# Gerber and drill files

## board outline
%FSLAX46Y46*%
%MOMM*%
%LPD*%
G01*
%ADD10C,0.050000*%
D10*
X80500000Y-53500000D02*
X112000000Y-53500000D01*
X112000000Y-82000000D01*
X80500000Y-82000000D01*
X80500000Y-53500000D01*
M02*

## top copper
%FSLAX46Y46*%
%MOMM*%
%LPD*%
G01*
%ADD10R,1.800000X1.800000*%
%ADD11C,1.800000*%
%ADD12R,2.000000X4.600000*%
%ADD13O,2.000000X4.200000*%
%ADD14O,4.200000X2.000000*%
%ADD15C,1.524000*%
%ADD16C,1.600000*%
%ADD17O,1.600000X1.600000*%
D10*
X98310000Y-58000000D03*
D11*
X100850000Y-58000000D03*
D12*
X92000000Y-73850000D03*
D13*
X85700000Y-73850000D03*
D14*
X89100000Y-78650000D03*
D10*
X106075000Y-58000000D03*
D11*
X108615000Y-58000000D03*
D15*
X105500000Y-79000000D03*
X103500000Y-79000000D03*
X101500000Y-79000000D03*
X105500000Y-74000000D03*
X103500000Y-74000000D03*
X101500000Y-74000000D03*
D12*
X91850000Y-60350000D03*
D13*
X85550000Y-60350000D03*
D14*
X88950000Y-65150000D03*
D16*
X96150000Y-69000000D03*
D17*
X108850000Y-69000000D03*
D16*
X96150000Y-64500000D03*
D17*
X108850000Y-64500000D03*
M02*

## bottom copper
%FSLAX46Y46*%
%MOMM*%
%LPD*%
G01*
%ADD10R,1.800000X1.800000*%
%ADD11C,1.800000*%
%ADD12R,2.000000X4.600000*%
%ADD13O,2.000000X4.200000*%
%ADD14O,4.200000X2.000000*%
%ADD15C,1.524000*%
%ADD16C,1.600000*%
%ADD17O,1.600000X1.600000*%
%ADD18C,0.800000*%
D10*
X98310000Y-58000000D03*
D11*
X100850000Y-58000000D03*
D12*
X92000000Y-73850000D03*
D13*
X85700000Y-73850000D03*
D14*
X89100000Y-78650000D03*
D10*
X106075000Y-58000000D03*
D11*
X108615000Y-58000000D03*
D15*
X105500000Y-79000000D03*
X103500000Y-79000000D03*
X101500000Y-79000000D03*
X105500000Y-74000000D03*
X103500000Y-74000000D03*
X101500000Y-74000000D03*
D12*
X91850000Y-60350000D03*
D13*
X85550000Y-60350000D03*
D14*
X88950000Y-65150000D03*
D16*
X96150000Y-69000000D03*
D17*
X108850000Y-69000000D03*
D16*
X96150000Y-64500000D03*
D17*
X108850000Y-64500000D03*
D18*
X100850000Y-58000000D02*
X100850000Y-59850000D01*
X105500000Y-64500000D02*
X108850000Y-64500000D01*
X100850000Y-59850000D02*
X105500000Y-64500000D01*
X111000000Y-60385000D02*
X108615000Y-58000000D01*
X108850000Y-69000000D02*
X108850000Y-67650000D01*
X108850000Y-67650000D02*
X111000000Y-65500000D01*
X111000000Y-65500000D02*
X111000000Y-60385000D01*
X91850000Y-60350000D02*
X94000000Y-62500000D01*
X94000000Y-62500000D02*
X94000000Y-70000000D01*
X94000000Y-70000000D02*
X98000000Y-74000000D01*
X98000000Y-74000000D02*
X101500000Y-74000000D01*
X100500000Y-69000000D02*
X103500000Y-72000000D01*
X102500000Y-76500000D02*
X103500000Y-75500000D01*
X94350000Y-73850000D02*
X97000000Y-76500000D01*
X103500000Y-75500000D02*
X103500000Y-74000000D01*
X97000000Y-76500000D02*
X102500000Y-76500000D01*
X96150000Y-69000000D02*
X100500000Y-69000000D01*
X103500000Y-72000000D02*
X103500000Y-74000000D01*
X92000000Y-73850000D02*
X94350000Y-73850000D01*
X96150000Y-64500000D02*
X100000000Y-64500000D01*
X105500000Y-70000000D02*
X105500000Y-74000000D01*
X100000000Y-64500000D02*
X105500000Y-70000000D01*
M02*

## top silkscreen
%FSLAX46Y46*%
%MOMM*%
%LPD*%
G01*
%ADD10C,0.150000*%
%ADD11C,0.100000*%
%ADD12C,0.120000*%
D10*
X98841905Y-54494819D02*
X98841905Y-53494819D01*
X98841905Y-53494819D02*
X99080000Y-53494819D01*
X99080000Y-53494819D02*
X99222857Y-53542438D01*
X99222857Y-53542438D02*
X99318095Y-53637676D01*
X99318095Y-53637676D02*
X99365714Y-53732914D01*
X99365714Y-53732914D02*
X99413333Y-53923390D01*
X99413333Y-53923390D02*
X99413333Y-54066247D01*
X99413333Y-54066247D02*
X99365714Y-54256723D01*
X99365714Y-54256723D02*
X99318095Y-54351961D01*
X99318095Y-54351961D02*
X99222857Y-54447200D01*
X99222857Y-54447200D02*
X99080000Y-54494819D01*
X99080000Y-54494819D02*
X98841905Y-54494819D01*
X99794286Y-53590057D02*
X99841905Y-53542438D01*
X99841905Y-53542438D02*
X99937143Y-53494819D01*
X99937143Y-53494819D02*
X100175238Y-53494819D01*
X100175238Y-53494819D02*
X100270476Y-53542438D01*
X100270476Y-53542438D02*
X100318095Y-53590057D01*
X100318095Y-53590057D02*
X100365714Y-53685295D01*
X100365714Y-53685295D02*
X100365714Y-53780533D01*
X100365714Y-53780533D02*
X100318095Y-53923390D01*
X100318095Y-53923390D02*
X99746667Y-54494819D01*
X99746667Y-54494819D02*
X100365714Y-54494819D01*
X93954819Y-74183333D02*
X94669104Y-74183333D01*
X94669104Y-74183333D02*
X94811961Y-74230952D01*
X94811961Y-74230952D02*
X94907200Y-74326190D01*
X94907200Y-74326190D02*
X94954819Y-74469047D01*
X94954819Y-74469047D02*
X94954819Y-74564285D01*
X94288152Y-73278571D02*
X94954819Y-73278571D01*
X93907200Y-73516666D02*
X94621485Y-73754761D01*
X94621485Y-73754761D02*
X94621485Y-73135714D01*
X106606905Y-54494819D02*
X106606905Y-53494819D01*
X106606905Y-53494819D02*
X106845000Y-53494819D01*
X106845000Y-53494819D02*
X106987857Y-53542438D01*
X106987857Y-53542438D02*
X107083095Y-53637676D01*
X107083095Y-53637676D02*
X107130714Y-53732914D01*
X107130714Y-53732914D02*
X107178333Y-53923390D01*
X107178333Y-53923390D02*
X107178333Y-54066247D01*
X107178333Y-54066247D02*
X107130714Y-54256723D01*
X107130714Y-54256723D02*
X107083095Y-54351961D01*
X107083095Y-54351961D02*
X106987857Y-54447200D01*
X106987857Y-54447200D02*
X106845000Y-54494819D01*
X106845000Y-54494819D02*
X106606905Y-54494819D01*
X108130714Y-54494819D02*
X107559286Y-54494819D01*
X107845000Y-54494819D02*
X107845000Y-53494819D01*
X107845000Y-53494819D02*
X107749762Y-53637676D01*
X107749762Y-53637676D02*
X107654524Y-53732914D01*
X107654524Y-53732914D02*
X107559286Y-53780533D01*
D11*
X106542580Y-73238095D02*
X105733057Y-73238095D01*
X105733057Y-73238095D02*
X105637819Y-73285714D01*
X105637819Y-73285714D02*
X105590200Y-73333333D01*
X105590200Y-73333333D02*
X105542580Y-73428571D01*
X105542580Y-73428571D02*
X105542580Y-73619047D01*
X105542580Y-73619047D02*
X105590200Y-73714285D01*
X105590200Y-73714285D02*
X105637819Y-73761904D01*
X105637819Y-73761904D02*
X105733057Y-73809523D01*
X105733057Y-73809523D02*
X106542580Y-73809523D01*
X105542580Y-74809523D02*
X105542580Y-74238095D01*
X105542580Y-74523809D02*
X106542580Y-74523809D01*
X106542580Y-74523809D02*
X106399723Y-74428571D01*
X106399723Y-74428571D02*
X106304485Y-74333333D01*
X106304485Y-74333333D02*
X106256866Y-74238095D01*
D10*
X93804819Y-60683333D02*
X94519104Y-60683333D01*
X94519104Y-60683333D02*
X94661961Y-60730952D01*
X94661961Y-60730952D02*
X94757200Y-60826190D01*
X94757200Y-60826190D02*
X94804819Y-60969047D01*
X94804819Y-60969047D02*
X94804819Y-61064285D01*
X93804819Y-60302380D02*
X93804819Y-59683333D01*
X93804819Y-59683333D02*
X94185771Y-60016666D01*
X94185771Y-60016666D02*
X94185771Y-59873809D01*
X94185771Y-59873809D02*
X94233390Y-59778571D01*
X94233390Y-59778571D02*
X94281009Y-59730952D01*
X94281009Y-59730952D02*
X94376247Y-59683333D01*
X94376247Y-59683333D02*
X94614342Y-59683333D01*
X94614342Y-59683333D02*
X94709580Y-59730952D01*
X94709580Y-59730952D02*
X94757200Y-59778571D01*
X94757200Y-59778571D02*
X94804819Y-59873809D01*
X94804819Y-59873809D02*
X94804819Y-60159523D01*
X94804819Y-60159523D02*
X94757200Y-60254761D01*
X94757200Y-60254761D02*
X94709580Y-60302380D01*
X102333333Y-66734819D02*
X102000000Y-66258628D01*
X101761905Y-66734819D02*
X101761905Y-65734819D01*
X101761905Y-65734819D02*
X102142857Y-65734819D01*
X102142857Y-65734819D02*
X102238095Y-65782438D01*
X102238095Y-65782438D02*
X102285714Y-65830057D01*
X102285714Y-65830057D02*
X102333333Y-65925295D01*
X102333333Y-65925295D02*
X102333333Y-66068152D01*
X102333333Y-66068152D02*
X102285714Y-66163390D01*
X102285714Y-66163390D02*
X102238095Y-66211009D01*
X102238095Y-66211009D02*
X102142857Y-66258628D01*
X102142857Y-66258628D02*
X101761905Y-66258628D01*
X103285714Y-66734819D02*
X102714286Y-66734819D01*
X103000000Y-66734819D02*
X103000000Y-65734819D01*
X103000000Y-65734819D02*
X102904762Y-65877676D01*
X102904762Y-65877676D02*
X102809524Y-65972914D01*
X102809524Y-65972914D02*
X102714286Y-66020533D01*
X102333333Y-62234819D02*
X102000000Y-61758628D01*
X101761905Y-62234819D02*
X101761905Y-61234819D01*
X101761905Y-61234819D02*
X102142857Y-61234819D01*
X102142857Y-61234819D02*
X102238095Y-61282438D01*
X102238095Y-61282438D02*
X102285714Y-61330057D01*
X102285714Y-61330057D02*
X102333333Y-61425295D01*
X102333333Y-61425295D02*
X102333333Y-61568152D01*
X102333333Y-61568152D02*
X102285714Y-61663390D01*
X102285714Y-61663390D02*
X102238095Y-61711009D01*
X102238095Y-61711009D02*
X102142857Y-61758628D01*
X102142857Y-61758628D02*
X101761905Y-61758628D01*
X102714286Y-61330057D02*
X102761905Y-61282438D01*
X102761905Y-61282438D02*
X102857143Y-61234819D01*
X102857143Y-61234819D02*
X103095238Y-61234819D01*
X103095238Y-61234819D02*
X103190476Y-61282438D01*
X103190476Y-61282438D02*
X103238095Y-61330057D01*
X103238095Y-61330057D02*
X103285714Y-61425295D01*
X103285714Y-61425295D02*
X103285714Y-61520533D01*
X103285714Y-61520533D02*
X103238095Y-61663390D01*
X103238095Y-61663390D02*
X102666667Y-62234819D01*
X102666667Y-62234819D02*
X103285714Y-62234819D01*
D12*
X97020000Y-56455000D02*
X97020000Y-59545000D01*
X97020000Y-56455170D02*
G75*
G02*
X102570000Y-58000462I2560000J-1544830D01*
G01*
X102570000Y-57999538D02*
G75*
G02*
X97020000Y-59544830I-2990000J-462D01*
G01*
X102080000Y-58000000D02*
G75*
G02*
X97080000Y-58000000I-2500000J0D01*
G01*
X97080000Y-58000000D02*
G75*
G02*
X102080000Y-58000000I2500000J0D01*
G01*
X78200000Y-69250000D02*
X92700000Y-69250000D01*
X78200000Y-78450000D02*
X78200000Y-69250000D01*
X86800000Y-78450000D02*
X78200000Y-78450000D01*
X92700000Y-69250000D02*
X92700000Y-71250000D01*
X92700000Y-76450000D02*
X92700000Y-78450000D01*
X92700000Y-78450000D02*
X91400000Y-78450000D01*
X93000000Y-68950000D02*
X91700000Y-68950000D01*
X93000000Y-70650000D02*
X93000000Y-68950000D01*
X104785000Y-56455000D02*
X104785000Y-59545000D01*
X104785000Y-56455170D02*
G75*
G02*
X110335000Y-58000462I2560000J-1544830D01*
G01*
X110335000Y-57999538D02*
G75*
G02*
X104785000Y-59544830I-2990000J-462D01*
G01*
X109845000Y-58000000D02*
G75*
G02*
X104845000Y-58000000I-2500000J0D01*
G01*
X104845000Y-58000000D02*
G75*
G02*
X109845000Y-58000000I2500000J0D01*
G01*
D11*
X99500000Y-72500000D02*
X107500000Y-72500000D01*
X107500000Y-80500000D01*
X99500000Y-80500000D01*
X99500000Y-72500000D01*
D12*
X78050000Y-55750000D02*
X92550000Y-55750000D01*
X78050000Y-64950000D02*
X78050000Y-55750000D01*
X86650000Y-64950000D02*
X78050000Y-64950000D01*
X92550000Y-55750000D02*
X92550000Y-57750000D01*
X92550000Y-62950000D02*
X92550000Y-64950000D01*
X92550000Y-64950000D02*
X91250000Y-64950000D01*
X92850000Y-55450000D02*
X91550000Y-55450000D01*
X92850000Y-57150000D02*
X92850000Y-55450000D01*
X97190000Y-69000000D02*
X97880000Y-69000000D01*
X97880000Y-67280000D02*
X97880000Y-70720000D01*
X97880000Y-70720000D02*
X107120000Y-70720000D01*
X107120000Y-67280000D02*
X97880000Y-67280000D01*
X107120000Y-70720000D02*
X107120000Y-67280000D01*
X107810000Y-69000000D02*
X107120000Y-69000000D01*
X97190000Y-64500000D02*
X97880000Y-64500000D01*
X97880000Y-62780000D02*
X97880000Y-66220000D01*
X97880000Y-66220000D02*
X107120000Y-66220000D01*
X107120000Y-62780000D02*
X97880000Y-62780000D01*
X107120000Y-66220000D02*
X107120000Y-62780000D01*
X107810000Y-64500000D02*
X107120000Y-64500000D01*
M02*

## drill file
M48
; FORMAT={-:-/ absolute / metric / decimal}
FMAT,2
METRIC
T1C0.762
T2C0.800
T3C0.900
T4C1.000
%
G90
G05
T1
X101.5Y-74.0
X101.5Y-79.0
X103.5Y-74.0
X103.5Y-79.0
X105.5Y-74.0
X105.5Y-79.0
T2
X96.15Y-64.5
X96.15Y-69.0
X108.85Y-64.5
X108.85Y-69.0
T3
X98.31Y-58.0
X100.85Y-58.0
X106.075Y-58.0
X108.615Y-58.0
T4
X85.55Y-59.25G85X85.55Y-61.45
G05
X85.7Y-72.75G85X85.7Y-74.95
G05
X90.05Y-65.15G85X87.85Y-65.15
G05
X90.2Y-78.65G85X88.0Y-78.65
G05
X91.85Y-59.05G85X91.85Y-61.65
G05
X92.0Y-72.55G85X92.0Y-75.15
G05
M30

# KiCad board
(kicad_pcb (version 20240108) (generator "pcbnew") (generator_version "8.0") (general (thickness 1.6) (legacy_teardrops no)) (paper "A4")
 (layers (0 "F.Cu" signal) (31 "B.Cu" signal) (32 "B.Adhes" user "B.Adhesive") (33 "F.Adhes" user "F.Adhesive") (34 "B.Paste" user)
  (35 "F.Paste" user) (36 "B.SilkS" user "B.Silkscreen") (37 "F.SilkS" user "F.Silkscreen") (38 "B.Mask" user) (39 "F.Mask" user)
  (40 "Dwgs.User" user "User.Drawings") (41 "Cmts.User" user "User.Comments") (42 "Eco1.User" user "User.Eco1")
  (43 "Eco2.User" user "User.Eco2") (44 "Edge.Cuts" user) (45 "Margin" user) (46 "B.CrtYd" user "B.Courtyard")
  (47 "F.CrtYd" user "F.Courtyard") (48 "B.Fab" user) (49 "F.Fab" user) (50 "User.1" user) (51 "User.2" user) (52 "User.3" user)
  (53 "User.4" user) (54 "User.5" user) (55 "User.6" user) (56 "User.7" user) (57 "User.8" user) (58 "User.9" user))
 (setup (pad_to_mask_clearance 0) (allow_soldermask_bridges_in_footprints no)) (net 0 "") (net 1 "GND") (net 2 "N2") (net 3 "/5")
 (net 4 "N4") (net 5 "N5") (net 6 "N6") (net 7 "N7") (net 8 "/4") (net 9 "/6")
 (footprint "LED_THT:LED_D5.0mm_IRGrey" (layer "F.Cu") (at 98.31 58)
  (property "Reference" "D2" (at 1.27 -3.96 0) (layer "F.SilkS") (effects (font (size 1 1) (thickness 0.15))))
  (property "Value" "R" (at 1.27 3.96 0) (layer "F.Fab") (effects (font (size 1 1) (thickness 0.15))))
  (fp_line (start -1.29 -1.545) (end -1.29 1.545) (stroke (width 0.12) (type solid)) (layer "F.SilkS"))
  (fp_arc (start -1.29 -1.54483) (mid 2.072002 -2.880433) (end 4.26 0.000462) (stroke (width 0.12) (type solid)) (layer "F.SilkS"))
  (fp_arc (start 4.26 -0.000462) (mid 2.072002 2.880433) (end -1.29 1.54483) (stroke (width 0.12) (type solid)) (layer "F.SilkS"))
  (fp_circle (center 1.27 0) (end 3.77 0) (stroke (width 0.12) (type solid)) (fill none) (layer "F.SilkS"))
  (pad "1" thru_hole rect (at 0 0) (size 1.8 1.8) (drill 0.9) (layers "*.Cu" "*.Mask") (remove_unused_layers no) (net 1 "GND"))
  (pad "2" thru_hole circle (at 2.54 0) (size 1.8 1.8) (drill 0.9) (layers "*.Cu" "*.Mask") (remove_unused_layers no) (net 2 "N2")))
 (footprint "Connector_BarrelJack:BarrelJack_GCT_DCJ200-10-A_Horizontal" (layer "F.Cu") (at 92 73.85 -90)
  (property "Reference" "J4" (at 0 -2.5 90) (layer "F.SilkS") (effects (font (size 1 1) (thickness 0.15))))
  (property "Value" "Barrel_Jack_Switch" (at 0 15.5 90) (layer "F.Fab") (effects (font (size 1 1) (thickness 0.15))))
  (fp_line (start -4.6 13.8) (end -4.6 -0.7) (stroke (width 0.12) (type solid)) (layer "F.SilkS"))
  (fp_line (start 4.6 13.8) (end -4.6 13.8) (stroke (width 0.12) (type solid)) (layer "F.SilkS"))
  (fp_line (start 4.6 5.2) (end 4.6 13.8) (stroke (width 0.12) (type solid)) (layer "F.SilkS"))
  (fp_line (start -4.6 -0.7) (end -2.6 -0.7) (stroke (width 0.12) (type solid)) (layer "F.SilkS"))
  (fp_line (start 2.6 -0.7) (end 4.6 -0.7) (stroke (width 0.12) (type solid)) (layer "F.SilkS"))
  (fp_line (start 4.6 -0.7) (end 4.6 0.6) (stroke (width 0.12) (type solid)) (layer "F.SilkS"))
  (fp_line (start -4.9 -1) (end -4.9 0.3) (stroke (width 0.12) (type solid)) (layer "F.SilkS"))
  (fp_line (start -3.2 -1) (end -4.9 -1) (stroke (width 0.12) (type solid)) (layer "F.SilkS"))
  (pad "1" thru_hole rect (at 0 0 270) (size 4.6 2) (drill oval 3.6 1) (layers "*.Cu" "*.Mask") (remove_unused_layers no) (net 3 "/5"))
  (pad "2" thru_hole oval (at 0 6.3 270) (size 4.2 2) (drill oval 3.2 1) (layers "*.Cu" "*.Mask") (remove_unused_layers no) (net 1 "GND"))
  (pad "3" thru_hole oval (at 4.8 2.9 270) (size 2 4.2) (drill oval 1 3.2) (layers "*.Cu" "*.Mask") (remove_unused_layers no) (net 1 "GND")))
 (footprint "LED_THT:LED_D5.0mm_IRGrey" (layer "F.Cu") (at 106.075 58)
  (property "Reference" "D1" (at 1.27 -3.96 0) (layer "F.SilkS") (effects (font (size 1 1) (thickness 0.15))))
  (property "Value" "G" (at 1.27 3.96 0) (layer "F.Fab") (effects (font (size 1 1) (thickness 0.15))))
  (fp_line (start -1.29 -1.545) (end -1.29 1.545) (stroke (width 0.12) (type solid)) (layer "F.SilkS"))
  (fp_arc (start -1.29 -1.54483) (mid 2.072002 -2.880433) (end 4.26 0.000462) (stroke (width 0.12) (type solid)) (layer "F.SilkS"))
  (fp_arc (start 4.26 -0.000462) (mid 2.072002 2.880433) (end -1.29 1.54483) (stroke (width 0.12) (type solid)) (layer "F.SilkS"))
  (fp_circle (center 1.27 0) (end 3.77 0) (stroke (width 0.12) (type solid)) (fill none) (layer "F.SilkS"))
  (pad "1" thru_hole rect (at 0 0) (size 1.8 1.8) (drill 0.9) (layers "*.Cu" "*.Mask") (remove_unused_layers no) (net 1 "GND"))
  (pad "2" thru_hole circle (at 2.54 0) (size 1.8 1.8) (drill 0.9) (layers "*.Cu" "*.Mask") (remove_unused_layers no) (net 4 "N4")))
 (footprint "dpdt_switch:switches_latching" (layer "F.Cu") (at 105.5 74 -90)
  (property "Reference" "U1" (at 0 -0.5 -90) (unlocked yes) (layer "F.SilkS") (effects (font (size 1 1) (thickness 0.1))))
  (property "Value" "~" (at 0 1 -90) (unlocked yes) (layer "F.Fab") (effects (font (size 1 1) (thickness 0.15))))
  (fp_rect (start -1.5 -2) (end 6.5 6) (stroke (width 0.1) (type solid)) (fill none) (layer "F.SilkS"))
  (pad "1" thru_hole circle (at 5 0 270) (size 1.524 1.524) (drill 0.762) (layers "*.Cu" "*.Mask") (remove_unused_layers no) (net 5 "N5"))
  (pad "2" thru_hole circle (at 5 2 270) (size 1.524 1.524) (drill 0.762) (layers "*.Cu" "*.Mask") (remove_unused_layers no) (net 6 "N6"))
  (pad "3" thru_hole circle (at 5 4 270) (size 1.524 1.524) (drill 0.762) (layers "*.Cu" "*.Mask") (remove_unused_layers no) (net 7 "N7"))
  (pad "4" thru_hole circle (at 0 0 270) (size 1.524 1.524) (drill 0.762) (layers "*.Cu" "*.Mask") (remove_unused_layers no) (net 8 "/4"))
  (pad "5" thru_hole circle (at 0 2 270) (size 1.524 1.524) (drill 0.762) (layers "*.Cu" "*.Mask") (remove_unused_layers no) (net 3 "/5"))
  (pad "6" thru_hole circle (at 0 4 270) (size 1.524 1.524) (drill 0.762) (layers "*.Cu" "*.Mask") (remove_unused_layers no) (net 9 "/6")))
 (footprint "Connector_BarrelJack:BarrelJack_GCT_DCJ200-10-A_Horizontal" (layer "F.Cu") (at 91.85 60.35 -90)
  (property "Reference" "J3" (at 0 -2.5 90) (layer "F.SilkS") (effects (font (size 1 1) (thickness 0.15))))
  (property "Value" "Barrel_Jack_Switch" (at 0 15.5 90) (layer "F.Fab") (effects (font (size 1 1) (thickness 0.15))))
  (fp_line (start -4.6 13.8) (end -4.6 -0.7) (stroke (width 0.12) (type solid)) (layer "F.SilkS"))
  (fp_line (start 4.6 13.8) (end -4.6 13.8) (stroke (width 0.12) (type solid)) (layer "F.SilkS"))
  (fp_line (start 4.6 5.2) (end 4.6 13.8) (stroke (width 0.12) (type solid)) (layer "F.SilkS"))
  (fp_line (start -4.6 -0.7) (end -2.6 -0.7) (stroke (width 0.12) (type solid)) (layer "F.SilkS"))
  (fp_line (start 2.6 -0.7) (end 4.6 -0.7) (stroke (width 0.12) (type solid)) (layer "F.SilkS"))
  (fp_line (start 4.6 -0.7) (end 4.6 0.6) (stroke (width 0.12) (type solid)) (layer "F.SilkS"))
  (fp_line (start -4.9 -1) (end -4.9 0.3) (stroke (width 0.12) (type solid)) (layer "F.SilkS"))
  (fp_line (start -3.2 -1) (end -4.9 -1) (stroke (width 0.12) (type solid)) (layer "F.SilkS"))
  (pad "1" thru_hole rect (at 0 0 270) (size 4.6 2) (drill oval 3.6 1) (layers "*.Cu" "*.Mask") (remove_unused_layers no) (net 9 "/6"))
  (pad "2" thru_hole oval (at 0 6.3 270) (size 4.2 2) (drill oval 3.2 1) (layers "*.Cu" "*.Mask") (remove_unused_layers no) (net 1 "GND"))
  (pad "3" thru_hole oval (at 4.8 2.9 270) (size 2 4.2) (drill oval 1 3.2) (layers "*.Cu" "*.Mask") (remove_unused_layers no) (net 1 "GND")))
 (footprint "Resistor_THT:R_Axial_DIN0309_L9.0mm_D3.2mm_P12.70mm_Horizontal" (layer "F.Cu") (at 96.15 69)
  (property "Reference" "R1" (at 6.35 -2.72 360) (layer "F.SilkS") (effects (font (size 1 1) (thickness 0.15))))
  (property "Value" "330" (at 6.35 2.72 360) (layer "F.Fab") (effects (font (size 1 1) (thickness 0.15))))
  (fp_line (start 1.04 0) (end 1.73 0) (stroke (width 0.12) (type solid)) (layer "F.SilkS"))
  (fp_line (start 1.73 -1.72) (end 1.73 1.72) (stroke (width 0.12) (type solid)) (layer "F.SilkS"))
  (fp_line (start 1.73 1.72) (end 10.97 1.72) (stroke (width 0.12) (type solid)) (layer "F.SilkS"))
  (fp_line (start 10.97 -1.72) (end 1.73 -1.72) (stroke (width 0.12) (type solid)) (layer "F.SilkS"))
  (fp_line (start 10.97 1.72) (end 10.97 -1.72) (stroke (width 0.12) (type solid)) (layer "F.SilkS"))
  (fp_line (start 11.66 0) (end 10.97 0) (stroke (width 0.12) (type solid)) (layer "F.SilkS"))
  (pad "1" thru_hole circle (at 0 0) (size 1.6 1.6) (drill 0.8) (layers "*.Cu" "*.Mask") (remove_unused_layers no) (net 3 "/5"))
  (pad "2" thru_hole oval (at 12.7 0) (size 1.6 1.6) (drill 0.8) (layers "*.Cu" "*.Mask") (remove_unused_layers no) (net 4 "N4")))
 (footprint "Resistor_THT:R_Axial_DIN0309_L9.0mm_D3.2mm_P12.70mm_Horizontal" (layer "F.Cu") (at 96.15 64.5)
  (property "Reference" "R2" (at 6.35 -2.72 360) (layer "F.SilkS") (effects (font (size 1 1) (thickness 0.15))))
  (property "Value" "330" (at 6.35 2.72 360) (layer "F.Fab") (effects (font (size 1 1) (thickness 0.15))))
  (fp_line (start 1.04 0) (end 1.73 0) (stroke (width 0.12) (type solid)) (layer "F.SilkS"))
  (fp_line (start 1.73 -1.72) (end 1.73 1.72) (stroke (width 0.12) (type solid)) (layer "F.SilkS"))
  (fp_line (start 1.73 1.72) (end 10.97 1.72) (stroke (width 0.12) (type solid)) (layer "F.SilkS"))
  (fp_line (start 10.97 -1.72) (end 1.73 -1.72) (stroke (width 0.12) (type solid)) (layer "F.SilkS"))
  (fp_line (start 10.97 1.72) (end 10.97 -1.72) (stroke (width 0.12) (type solid)) (layer "F.SilkS"))
  (fp_line (start 11.66 0) (end 10.97 0) (stroke (width 0.12) (type solid)) (layer "F.SilkS"))
  (pad "1" thru_hole circle (at 0 0) (size 1.6 1.6) (drill 0.8) (layers "*.Cu" "*.Mask") (remove_unused_layers no) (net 8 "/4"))
  (pad "2" thru_hole oval (at 12.7 0) (size 1.6 1.6) (drill 0.8) (layers "*.Cu" "*.Mask") (remove_unused_layers no) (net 2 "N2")))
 (gr_rect (start 80.5 53.5) (end 112 82) (stroke (width 0.05) (type default)) (fill none) (layer "Edge.Cuts"))
 (segment (start 100.85 58) (end 100.85 59.85) (width 0.8) (layer "B.Cu") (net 2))
 (segment (start 105.5 64.5) (end 108.85 64.5) (width 0.8) (layer "B.Cu") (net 2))
 (segment (start 100.85 59.85) (end 105.5 64.5) (width 0.8) (layer "B.Cu") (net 2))
 (segment (start 111 60.385) (end 108.615 58) (width 0.8) (layer "B.Cu") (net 4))
 (segment (start 108.85 69) (end 108.85 67.65) (width 0.8) (layer "B.Cu") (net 4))
 (segment (start 108.85 67.65) (end 111 65.5) (width 0.8) (layer "B.Cu") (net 4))
 (segment (start 111 65.5) (end 111 60.385) (width 0.8) (layer "B.Cu") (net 4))
 (segment (start 91.85 60.35) (end 94 62.5) (width 0.8) (layer "B.Cu") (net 9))
 (segment (start 94 62.5) (end 94 70) (width 0.8) (layer "B.Cu") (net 9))
 (segment (start 94 70) (end 98 74) (width 0.8) (layer "B.Cu") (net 9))
 (segment (start 98 74) (end 101.5 74) (width 0.8) (layer "B.Cu") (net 9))
 (segment (start 100.5 69) (end 103.5 72) (width 0.8) (layer "B.Cu") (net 3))
 (segment (start 102.5 76.5) (end 103.5 75.5) (width 0.8) (layer "B.Cu") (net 3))
 (segment (start 94.35 73.85) (end 97 76.5) (width 0.8) (layer "B.Cu") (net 3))
 (segment (start 103.5 75.5) (end 103.5 74) (width 0.8) (layer "B.Cu") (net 3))
 (segment (start 97 76.5) (end 102.5 76.5) (width 0.8) (layer "B.Cu") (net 3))
 (segment (start 96.15 69) (end 100.5 69) (width 0.8) (layer "B.Cu") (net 3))
 (segment (start 103.5 72) (end 103.5 74) (width 0.8) (layer "B.Cu") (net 3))
 (segment (start 92 73.85) (end 94.35 73.85) (width 0.8) (layer "B.Cu") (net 3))
 (segment (start 96.15 64.5) (end 100 64.5) (width 0.8) (layer "B.Cu") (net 8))
 (segment (start 105.5 70) (end 105.5 74) (width 0.8) (layer "B.Cu") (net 8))
 (segment (start 100 64.5) (end 105.5 70) (width 0.8) (layer "B.Cu") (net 8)))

